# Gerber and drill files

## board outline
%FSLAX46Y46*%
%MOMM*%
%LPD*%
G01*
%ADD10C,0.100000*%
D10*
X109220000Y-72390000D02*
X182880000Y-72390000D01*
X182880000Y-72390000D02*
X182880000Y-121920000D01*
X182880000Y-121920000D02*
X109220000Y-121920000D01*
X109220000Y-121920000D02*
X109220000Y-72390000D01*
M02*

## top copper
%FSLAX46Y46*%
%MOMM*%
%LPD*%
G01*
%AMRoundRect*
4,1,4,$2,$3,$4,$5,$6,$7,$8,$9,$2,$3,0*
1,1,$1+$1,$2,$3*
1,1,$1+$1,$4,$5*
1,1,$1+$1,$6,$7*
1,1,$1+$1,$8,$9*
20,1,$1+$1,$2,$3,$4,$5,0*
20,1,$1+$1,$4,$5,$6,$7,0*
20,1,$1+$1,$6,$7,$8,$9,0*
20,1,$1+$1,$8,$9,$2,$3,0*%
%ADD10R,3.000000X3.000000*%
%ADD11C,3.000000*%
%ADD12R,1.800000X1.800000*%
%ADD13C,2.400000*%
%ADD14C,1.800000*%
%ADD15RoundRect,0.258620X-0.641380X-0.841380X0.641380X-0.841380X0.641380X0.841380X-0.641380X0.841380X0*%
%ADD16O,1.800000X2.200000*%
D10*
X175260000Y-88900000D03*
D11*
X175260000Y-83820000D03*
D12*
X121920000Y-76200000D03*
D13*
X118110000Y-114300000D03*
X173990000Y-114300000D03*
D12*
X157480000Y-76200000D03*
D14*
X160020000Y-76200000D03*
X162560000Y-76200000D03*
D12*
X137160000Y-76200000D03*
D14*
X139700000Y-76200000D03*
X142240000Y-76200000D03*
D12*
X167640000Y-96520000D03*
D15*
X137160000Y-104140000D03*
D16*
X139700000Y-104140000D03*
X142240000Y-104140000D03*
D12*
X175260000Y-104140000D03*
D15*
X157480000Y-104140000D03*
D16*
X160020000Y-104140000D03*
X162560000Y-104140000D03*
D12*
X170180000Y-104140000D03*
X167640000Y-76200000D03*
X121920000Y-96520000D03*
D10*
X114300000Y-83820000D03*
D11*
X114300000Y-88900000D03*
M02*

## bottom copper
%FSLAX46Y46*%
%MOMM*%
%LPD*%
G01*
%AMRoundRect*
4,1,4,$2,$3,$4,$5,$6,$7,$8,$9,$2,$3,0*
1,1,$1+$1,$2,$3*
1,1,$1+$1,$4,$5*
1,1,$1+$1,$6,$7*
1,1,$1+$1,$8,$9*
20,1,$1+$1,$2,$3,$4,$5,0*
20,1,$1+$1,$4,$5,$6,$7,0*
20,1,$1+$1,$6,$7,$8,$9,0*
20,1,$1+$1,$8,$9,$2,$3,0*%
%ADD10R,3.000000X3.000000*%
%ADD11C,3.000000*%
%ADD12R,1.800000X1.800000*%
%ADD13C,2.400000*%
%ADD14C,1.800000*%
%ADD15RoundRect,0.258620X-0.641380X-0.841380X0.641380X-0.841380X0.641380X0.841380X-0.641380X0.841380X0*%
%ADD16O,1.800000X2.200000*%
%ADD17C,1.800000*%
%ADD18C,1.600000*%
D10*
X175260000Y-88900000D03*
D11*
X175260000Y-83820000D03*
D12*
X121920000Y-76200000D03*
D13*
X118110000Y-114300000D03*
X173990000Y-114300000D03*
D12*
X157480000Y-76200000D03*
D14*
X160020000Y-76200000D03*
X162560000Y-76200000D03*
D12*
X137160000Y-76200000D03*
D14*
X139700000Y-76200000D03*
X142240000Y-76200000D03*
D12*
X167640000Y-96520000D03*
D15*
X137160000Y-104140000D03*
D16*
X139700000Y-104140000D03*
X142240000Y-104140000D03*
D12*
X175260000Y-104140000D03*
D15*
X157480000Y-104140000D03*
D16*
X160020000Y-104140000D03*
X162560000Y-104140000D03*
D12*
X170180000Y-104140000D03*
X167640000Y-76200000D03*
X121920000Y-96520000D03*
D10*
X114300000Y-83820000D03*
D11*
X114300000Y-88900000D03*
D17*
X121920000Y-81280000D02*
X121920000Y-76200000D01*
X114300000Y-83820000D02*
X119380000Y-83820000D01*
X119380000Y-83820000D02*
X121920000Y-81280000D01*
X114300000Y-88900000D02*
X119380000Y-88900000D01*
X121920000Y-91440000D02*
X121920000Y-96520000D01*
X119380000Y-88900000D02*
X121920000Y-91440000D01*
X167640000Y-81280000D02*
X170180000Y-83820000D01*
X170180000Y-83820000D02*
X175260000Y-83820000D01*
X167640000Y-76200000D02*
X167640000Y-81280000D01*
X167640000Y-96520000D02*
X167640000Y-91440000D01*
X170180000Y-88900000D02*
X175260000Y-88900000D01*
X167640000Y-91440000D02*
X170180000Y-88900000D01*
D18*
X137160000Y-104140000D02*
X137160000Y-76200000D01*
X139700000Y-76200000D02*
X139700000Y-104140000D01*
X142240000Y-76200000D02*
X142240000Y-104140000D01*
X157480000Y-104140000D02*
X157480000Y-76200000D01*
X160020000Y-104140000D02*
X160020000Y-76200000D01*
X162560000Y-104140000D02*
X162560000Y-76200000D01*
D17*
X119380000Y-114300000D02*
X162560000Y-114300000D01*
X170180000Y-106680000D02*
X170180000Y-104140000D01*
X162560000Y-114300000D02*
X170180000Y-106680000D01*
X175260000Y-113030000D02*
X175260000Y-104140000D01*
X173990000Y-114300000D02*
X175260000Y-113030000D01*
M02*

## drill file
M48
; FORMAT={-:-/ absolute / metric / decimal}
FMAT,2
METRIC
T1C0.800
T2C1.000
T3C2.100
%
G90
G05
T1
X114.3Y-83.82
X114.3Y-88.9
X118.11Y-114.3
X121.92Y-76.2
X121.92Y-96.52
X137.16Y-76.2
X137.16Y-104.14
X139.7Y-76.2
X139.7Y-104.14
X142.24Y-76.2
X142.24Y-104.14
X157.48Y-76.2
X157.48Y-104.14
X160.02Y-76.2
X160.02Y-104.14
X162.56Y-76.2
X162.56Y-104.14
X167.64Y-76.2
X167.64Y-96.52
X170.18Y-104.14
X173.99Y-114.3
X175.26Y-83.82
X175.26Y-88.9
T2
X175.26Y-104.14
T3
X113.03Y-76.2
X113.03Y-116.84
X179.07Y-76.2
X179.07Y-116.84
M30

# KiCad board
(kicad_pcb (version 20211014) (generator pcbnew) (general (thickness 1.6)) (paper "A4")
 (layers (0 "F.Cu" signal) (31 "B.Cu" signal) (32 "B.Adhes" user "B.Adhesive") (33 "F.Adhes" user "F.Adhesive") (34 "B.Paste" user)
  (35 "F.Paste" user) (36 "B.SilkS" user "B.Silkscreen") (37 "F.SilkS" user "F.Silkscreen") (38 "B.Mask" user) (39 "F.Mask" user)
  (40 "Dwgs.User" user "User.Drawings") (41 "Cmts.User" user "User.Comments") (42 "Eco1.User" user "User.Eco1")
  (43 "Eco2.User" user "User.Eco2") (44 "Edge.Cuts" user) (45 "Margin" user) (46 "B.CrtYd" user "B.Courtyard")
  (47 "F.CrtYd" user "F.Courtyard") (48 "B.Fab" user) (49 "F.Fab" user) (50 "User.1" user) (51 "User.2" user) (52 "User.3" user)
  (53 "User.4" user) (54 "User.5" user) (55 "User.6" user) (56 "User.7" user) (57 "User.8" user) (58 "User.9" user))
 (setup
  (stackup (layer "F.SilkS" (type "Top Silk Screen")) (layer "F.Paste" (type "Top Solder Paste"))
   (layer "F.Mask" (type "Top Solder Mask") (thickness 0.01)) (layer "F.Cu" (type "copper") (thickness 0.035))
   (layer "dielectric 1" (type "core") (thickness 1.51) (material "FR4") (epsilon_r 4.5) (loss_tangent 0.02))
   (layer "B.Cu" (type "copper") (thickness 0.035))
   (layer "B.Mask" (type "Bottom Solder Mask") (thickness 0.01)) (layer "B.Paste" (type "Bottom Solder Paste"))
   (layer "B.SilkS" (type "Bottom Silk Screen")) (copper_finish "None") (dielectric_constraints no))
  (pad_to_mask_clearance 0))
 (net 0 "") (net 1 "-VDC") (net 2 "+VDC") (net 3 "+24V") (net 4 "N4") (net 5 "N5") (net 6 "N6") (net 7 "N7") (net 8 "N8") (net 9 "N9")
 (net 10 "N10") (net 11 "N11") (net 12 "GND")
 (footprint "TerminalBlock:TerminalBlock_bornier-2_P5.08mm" (layer "F.Cu") (at 175.26 88.9 90)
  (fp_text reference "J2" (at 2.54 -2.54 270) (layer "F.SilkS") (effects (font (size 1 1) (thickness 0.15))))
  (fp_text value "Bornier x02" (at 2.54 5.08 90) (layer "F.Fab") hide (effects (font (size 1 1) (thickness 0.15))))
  (pad "1" thru_hole rect (at 0 0 90) (size 3 3) (drill 0.8) (layers *.Cu *.Mask) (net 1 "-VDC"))
  (pad "2" thru_hole circle (at 5.08 0 90) (size 3 3) (drill 0.8) (layers *.Cu *.Mask) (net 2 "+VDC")))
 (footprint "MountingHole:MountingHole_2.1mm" (layer "F.Cu") (at 179.07 116.84)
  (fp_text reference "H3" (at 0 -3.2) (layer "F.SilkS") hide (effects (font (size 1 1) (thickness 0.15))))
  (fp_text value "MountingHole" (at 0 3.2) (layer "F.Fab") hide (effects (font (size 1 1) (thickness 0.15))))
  (pad "" np_thru_hole circle (at 0 0) (size 2.1 2.1) (drill 2.1) (layers *.Cu *.Mask)))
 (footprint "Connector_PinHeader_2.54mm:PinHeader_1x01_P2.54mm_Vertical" (layer "F.Cu") (at 121.92 76.2)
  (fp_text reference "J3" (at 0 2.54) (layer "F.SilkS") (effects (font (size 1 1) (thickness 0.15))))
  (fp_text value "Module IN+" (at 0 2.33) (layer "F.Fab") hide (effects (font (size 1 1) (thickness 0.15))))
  (pad "1" thru_hole rect (at 0 0) (size 1.8 1.8) (drill 0.8) (layers *.Cu *.Mask) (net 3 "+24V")))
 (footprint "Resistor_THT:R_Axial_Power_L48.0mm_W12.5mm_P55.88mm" (layer "F.Cu") (at 118.11 114.3)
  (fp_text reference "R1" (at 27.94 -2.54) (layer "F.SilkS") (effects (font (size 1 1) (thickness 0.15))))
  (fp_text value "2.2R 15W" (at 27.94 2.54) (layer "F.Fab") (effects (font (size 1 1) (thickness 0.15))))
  (pad "1" thru_hole circle (at 0 0) (size 2.4 2.4) (drill 0.8) (layers *.Cu *.Mask) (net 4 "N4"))
  (pad "2" thru_hole circle (at 55.88 0) (size 2.4 2.4) (drill 0.8) (layers *.Cu *.Mask) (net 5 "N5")))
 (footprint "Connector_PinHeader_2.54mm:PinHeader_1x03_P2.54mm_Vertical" (layer "F.Cu") (at 157.48 76.2 90)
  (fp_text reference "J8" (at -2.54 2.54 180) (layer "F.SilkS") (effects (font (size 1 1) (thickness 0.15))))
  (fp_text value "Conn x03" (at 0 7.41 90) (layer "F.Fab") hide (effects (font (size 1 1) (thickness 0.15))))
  (pad "1" thru_hole rect (at 0 0 90) (size 1.8 1.8) (drill 0.8) (layers *.Cu *.Mask) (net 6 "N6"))
  (pad "2" thru_hole circle (at 0 2.54 90) (size 1.8 1.8) (drill 0.8) (layers *.Cu *.Mask) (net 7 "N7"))
  (pad "3" thru_hole circle (at 0 5.08 90) (size 1.8 1.8) (drill 0.8) (layers *.Cu *.Mask) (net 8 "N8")))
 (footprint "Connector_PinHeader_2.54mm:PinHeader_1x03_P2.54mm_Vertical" (layer "F.Cu") (at 137.16 76.2 90)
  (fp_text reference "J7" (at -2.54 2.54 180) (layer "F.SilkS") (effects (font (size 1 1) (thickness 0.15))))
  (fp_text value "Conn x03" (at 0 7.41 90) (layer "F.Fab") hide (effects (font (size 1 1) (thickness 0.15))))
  (pad "1" thru_hole rect (at 0 0 90) (size 1.8 1.8) (drill 0.8) (layers *.Cu *.Mask) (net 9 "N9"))
  (pad "2" thru_hole circle (at 0 2.54 90) (size 1.8 1.8) (drill 0.8) (layers *.Cu *.Mask) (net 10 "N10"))
  (pad "3" thru_hole circle (at 0 5.08 90) (size 1.8 1.8) (drill 0.8) (layers *.Cu *.Mask) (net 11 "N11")))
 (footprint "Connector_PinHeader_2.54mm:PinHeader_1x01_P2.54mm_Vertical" (layer "F.Cu") (at 167.64 96.52)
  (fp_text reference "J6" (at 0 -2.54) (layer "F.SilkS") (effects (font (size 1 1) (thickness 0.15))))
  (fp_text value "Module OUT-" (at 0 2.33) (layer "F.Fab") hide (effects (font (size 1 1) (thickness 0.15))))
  (pad "1" thru_hole rect (at 0 0) (size 1.8 1.8) (drill 0.8) (layers *.Cu *.Mask) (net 1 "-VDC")))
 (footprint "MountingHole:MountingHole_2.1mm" (layer "F.Cu") (at 113.03 116.84)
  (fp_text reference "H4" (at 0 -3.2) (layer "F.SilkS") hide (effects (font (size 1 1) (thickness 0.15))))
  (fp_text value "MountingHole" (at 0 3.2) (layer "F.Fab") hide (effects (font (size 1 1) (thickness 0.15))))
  (pad "" np_thru_hole circle (at 0 0) (size 2.1 2.1) (drill 2.1) (layers *.Cu *.Mask)))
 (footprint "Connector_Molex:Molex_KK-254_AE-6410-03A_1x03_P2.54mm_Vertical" (layer "F.Cu") (at 137.16 104.14)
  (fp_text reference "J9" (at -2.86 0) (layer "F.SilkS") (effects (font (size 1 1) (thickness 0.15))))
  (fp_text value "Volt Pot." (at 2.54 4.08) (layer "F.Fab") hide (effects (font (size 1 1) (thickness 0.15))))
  (pad "1" thru_hole roundrect (at 0 0) (size 1.8 2.2) (drill 0.8) (layers *.Cu *.Mask) (roundrect_rratio 0.143678) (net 9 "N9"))
  (pad "2" thru_hole oval (at 2.54 0) (size 1.8 2.2) (drill 0.8) (layers *.Cu *.Mask) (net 10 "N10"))
  (pad "3" thru_hole oval (at 5.08 0) (size 1.8 2.2) (drill 0.8) (layers *.Cu *.Mask) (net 11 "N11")))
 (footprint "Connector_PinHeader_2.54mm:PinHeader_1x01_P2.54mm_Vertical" (layer "F.Cu") (at 175.26 104.14)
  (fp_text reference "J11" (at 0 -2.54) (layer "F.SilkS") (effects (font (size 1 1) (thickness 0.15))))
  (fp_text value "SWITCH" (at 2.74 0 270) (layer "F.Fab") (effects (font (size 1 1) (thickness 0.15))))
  (pad "1" thru_hole rect (at 0 0) (size 1.8 1.8) (drill 1) (layers *.Cu *.Mask) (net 5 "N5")))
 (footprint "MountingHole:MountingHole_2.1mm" (layer "F.Cu") (at 179.07 76.2)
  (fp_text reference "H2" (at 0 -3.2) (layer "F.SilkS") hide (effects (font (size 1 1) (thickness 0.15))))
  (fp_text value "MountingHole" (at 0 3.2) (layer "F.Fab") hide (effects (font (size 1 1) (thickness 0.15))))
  (pad "" np_thru_hole circle (at 0 0) (size 2.1 2.1) (drill 2.1) (layers *.Cu *.Mask)))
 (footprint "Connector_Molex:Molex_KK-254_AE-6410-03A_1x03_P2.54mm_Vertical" (layer "F.Cu") (at 157.48 104.14)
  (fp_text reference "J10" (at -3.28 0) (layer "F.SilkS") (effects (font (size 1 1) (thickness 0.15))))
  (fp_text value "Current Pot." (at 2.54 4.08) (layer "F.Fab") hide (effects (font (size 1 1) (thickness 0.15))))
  (pad "1" thru_hole roundrect (at 0 0) (size 1.8 2.2) (drill 0.8) (layers *.Cu *.Mask) (roundrect_rratio 0.143678) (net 6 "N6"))
  (pad "2" thru_hole oval (at 2.54 0) (size 1.8 2.2) (drill 0.8) (layers *.Cu *.Mask) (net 7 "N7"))
  (pad "3" thru_hole oval (at 5.08 0) (size 1.8 2.2) (drill 0.8) (layers *.Cu *.Mask) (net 8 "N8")))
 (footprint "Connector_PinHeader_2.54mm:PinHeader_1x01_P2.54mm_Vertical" (layer "F.Cu") (at 170.18 104.14)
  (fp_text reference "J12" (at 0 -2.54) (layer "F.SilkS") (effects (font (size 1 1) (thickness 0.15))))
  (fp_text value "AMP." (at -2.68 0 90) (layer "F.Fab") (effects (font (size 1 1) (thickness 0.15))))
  (pad "1" thru_hole rect (at 0 0) (size 1.8 1.8) (drill 0.8) (layers *.Cu *.Mask) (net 4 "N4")))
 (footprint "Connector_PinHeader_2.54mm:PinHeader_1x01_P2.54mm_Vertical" (layer "F.Cu") (at 167.64 76.2)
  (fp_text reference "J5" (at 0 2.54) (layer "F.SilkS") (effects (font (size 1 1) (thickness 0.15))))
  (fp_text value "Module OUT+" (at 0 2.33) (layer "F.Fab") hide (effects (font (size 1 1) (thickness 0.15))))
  (pad "1" thru_hole rect (at 0 0) (size 1.8 1.8) (drill 0.8) (layers *.Cu *.Mask) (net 2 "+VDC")))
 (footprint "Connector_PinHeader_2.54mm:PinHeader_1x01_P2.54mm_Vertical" (layer "F.Cu") (at 121.92 96.52)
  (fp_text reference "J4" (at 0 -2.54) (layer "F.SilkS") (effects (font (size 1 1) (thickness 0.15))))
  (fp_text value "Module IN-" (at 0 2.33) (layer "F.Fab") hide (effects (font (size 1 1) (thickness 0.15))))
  (pad "1" thru_hole rect (at 0 0) (size 1.8 1.8) (drill 0.8) (layers *.Cu *.Mask) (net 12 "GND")))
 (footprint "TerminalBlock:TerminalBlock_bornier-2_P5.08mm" (layer "F.Cu") (at 114.3 83.82 -90)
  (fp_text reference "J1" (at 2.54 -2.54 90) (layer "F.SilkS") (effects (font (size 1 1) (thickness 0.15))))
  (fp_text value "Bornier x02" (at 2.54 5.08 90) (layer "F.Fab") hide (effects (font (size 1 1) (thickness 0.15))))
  (pad "1" thru_hole rect (at 0 0 270) (size 3 3) (drill 0.8) (layers *.Cu *.Mask) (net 3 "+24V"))
  (pad "2" thru_hole circle (at 5.08 0 270) (size 3 3) (drill 0.8) (layers *.Cu *.Mask) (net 12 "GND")))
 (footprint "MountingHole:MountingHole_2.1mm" (layer "F.Cu") (at 113.03 76.2)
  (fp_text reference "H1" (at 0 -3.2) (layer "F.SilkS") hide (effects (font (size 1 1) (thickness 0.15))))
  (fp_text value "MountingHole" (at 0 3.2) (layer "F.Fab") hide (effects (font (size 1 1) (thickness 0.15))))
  (pad "" np_thru_hole circle (at 0 0) (size 2.1 2.1) (drill 2.1) (layers *.Cu *.Mask)))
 (gr_line (start 109.22 72.39) (end 182.88 72.39) (layer "Edge.Cuts") (width 0.1))
 (gr_line (start 182.88 72.39) (end 182.88 121.92) (layer "Edge.Cuts") (width 0.1))
 (gr_line (start 182.88 121.92) (end 109.22 121.92) (layer "Edge.Cuts") (width 0.1))
 (gr_line (start 109.22 121.92) (end 109.22 72.39) (layer "Edge.Cuts") (width 0.1))
 (segment (start 121.92 81.28) (end 121.92 76.2) (width 1.8) (layer "B.Cu") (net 3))
 (segment (start 114.3 83.82) (end 119.38 83.82) (width 1.8) (layer "B.Cu") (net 3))
 (segment (start 119.38 83.82) (end 121.92 81.28) (width 1.8) (layer "B.Cu") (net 3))
 (segment (start 114.3 88.9) (end 119.38 88.9) (width 1.8) (layer "B.Cu") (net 12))
 (segment (start 121.92 91.44) (end 121.92 96.52) (width 1.8) (layer "B.Cu") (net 12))
 (segment (start 119.38 88.9) (end 121.92 91.44) (width 1.8) (layer "B.Cu") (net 12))
 (segment (start 167.64 81.28) (end 170.18 83.82) (width 1.8) (layer "B.Cu") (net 2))
 (segment (start 170.18 83.82) (end 175.26 83.82) (width 1.8) (layer "B.Cu") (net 2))
 (segment (start 167.64 76.2) (end 167.64 81.28) (width 1.8) (layer "B.Cu") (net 2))
 (segment (start 167.64 96.52) (end 167.64 91.44) (width 1.8) (layer "B.Cu") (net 1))
 (segment (start 170.18 88.9) (end 175.26 88.9) (width 1.8) (layer "B.Cu") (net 1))
 (segment (start 167.64 91.44) (end 170.18 88.9) (width 1.8) (layer "B.Cu") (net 1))
 (segment (start 137.16 104.14) (end 137.16 76.2) (width 1.6) (layer "B.Cu") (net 9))
 (segment (start 139.7 76.2) (end 139.7 104.14) (width 1.6) (layer "B.Cu") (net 10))
 (segment (start 142.24 76.2) (end 142.24 104.14) (width 1.6) (layer "B.Cu") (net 11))
 (segment (start 157.48 104.14) (end 157.48 76.2) (width 1.6) (layer "B.Cu") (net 6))
 (segment (start 160.02 104.14) (end 160.02 76.2) (width 1.6) (layer "B.Cu") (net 7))
 (segment (start 162.56 104.14) (end 162.56 76.2) (width 1.6) (layer "B.Cu") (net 8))
 (segment (start 119.38 114.3) (end 162.56 114.3) (width 1.8) (layer "B.Cu") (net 4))
 (segment (start 170.18 106.68) (end 170.18 104.14) (width 1.8) (layer "B.Cu") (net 4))
 (segment (start 162.56 114.3) (end 170.18 106.68) (width 1.8) (layer "B.Cu") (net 4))
 (segment (start 175.26 113.03) (end 175.26 104.14) (width 1.8) (layer "B.Cu") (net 5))
 (segment (start 173.99 114.3) (end 175.26 113.03) (width 1.8) (layer "B.Cu") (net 5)))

